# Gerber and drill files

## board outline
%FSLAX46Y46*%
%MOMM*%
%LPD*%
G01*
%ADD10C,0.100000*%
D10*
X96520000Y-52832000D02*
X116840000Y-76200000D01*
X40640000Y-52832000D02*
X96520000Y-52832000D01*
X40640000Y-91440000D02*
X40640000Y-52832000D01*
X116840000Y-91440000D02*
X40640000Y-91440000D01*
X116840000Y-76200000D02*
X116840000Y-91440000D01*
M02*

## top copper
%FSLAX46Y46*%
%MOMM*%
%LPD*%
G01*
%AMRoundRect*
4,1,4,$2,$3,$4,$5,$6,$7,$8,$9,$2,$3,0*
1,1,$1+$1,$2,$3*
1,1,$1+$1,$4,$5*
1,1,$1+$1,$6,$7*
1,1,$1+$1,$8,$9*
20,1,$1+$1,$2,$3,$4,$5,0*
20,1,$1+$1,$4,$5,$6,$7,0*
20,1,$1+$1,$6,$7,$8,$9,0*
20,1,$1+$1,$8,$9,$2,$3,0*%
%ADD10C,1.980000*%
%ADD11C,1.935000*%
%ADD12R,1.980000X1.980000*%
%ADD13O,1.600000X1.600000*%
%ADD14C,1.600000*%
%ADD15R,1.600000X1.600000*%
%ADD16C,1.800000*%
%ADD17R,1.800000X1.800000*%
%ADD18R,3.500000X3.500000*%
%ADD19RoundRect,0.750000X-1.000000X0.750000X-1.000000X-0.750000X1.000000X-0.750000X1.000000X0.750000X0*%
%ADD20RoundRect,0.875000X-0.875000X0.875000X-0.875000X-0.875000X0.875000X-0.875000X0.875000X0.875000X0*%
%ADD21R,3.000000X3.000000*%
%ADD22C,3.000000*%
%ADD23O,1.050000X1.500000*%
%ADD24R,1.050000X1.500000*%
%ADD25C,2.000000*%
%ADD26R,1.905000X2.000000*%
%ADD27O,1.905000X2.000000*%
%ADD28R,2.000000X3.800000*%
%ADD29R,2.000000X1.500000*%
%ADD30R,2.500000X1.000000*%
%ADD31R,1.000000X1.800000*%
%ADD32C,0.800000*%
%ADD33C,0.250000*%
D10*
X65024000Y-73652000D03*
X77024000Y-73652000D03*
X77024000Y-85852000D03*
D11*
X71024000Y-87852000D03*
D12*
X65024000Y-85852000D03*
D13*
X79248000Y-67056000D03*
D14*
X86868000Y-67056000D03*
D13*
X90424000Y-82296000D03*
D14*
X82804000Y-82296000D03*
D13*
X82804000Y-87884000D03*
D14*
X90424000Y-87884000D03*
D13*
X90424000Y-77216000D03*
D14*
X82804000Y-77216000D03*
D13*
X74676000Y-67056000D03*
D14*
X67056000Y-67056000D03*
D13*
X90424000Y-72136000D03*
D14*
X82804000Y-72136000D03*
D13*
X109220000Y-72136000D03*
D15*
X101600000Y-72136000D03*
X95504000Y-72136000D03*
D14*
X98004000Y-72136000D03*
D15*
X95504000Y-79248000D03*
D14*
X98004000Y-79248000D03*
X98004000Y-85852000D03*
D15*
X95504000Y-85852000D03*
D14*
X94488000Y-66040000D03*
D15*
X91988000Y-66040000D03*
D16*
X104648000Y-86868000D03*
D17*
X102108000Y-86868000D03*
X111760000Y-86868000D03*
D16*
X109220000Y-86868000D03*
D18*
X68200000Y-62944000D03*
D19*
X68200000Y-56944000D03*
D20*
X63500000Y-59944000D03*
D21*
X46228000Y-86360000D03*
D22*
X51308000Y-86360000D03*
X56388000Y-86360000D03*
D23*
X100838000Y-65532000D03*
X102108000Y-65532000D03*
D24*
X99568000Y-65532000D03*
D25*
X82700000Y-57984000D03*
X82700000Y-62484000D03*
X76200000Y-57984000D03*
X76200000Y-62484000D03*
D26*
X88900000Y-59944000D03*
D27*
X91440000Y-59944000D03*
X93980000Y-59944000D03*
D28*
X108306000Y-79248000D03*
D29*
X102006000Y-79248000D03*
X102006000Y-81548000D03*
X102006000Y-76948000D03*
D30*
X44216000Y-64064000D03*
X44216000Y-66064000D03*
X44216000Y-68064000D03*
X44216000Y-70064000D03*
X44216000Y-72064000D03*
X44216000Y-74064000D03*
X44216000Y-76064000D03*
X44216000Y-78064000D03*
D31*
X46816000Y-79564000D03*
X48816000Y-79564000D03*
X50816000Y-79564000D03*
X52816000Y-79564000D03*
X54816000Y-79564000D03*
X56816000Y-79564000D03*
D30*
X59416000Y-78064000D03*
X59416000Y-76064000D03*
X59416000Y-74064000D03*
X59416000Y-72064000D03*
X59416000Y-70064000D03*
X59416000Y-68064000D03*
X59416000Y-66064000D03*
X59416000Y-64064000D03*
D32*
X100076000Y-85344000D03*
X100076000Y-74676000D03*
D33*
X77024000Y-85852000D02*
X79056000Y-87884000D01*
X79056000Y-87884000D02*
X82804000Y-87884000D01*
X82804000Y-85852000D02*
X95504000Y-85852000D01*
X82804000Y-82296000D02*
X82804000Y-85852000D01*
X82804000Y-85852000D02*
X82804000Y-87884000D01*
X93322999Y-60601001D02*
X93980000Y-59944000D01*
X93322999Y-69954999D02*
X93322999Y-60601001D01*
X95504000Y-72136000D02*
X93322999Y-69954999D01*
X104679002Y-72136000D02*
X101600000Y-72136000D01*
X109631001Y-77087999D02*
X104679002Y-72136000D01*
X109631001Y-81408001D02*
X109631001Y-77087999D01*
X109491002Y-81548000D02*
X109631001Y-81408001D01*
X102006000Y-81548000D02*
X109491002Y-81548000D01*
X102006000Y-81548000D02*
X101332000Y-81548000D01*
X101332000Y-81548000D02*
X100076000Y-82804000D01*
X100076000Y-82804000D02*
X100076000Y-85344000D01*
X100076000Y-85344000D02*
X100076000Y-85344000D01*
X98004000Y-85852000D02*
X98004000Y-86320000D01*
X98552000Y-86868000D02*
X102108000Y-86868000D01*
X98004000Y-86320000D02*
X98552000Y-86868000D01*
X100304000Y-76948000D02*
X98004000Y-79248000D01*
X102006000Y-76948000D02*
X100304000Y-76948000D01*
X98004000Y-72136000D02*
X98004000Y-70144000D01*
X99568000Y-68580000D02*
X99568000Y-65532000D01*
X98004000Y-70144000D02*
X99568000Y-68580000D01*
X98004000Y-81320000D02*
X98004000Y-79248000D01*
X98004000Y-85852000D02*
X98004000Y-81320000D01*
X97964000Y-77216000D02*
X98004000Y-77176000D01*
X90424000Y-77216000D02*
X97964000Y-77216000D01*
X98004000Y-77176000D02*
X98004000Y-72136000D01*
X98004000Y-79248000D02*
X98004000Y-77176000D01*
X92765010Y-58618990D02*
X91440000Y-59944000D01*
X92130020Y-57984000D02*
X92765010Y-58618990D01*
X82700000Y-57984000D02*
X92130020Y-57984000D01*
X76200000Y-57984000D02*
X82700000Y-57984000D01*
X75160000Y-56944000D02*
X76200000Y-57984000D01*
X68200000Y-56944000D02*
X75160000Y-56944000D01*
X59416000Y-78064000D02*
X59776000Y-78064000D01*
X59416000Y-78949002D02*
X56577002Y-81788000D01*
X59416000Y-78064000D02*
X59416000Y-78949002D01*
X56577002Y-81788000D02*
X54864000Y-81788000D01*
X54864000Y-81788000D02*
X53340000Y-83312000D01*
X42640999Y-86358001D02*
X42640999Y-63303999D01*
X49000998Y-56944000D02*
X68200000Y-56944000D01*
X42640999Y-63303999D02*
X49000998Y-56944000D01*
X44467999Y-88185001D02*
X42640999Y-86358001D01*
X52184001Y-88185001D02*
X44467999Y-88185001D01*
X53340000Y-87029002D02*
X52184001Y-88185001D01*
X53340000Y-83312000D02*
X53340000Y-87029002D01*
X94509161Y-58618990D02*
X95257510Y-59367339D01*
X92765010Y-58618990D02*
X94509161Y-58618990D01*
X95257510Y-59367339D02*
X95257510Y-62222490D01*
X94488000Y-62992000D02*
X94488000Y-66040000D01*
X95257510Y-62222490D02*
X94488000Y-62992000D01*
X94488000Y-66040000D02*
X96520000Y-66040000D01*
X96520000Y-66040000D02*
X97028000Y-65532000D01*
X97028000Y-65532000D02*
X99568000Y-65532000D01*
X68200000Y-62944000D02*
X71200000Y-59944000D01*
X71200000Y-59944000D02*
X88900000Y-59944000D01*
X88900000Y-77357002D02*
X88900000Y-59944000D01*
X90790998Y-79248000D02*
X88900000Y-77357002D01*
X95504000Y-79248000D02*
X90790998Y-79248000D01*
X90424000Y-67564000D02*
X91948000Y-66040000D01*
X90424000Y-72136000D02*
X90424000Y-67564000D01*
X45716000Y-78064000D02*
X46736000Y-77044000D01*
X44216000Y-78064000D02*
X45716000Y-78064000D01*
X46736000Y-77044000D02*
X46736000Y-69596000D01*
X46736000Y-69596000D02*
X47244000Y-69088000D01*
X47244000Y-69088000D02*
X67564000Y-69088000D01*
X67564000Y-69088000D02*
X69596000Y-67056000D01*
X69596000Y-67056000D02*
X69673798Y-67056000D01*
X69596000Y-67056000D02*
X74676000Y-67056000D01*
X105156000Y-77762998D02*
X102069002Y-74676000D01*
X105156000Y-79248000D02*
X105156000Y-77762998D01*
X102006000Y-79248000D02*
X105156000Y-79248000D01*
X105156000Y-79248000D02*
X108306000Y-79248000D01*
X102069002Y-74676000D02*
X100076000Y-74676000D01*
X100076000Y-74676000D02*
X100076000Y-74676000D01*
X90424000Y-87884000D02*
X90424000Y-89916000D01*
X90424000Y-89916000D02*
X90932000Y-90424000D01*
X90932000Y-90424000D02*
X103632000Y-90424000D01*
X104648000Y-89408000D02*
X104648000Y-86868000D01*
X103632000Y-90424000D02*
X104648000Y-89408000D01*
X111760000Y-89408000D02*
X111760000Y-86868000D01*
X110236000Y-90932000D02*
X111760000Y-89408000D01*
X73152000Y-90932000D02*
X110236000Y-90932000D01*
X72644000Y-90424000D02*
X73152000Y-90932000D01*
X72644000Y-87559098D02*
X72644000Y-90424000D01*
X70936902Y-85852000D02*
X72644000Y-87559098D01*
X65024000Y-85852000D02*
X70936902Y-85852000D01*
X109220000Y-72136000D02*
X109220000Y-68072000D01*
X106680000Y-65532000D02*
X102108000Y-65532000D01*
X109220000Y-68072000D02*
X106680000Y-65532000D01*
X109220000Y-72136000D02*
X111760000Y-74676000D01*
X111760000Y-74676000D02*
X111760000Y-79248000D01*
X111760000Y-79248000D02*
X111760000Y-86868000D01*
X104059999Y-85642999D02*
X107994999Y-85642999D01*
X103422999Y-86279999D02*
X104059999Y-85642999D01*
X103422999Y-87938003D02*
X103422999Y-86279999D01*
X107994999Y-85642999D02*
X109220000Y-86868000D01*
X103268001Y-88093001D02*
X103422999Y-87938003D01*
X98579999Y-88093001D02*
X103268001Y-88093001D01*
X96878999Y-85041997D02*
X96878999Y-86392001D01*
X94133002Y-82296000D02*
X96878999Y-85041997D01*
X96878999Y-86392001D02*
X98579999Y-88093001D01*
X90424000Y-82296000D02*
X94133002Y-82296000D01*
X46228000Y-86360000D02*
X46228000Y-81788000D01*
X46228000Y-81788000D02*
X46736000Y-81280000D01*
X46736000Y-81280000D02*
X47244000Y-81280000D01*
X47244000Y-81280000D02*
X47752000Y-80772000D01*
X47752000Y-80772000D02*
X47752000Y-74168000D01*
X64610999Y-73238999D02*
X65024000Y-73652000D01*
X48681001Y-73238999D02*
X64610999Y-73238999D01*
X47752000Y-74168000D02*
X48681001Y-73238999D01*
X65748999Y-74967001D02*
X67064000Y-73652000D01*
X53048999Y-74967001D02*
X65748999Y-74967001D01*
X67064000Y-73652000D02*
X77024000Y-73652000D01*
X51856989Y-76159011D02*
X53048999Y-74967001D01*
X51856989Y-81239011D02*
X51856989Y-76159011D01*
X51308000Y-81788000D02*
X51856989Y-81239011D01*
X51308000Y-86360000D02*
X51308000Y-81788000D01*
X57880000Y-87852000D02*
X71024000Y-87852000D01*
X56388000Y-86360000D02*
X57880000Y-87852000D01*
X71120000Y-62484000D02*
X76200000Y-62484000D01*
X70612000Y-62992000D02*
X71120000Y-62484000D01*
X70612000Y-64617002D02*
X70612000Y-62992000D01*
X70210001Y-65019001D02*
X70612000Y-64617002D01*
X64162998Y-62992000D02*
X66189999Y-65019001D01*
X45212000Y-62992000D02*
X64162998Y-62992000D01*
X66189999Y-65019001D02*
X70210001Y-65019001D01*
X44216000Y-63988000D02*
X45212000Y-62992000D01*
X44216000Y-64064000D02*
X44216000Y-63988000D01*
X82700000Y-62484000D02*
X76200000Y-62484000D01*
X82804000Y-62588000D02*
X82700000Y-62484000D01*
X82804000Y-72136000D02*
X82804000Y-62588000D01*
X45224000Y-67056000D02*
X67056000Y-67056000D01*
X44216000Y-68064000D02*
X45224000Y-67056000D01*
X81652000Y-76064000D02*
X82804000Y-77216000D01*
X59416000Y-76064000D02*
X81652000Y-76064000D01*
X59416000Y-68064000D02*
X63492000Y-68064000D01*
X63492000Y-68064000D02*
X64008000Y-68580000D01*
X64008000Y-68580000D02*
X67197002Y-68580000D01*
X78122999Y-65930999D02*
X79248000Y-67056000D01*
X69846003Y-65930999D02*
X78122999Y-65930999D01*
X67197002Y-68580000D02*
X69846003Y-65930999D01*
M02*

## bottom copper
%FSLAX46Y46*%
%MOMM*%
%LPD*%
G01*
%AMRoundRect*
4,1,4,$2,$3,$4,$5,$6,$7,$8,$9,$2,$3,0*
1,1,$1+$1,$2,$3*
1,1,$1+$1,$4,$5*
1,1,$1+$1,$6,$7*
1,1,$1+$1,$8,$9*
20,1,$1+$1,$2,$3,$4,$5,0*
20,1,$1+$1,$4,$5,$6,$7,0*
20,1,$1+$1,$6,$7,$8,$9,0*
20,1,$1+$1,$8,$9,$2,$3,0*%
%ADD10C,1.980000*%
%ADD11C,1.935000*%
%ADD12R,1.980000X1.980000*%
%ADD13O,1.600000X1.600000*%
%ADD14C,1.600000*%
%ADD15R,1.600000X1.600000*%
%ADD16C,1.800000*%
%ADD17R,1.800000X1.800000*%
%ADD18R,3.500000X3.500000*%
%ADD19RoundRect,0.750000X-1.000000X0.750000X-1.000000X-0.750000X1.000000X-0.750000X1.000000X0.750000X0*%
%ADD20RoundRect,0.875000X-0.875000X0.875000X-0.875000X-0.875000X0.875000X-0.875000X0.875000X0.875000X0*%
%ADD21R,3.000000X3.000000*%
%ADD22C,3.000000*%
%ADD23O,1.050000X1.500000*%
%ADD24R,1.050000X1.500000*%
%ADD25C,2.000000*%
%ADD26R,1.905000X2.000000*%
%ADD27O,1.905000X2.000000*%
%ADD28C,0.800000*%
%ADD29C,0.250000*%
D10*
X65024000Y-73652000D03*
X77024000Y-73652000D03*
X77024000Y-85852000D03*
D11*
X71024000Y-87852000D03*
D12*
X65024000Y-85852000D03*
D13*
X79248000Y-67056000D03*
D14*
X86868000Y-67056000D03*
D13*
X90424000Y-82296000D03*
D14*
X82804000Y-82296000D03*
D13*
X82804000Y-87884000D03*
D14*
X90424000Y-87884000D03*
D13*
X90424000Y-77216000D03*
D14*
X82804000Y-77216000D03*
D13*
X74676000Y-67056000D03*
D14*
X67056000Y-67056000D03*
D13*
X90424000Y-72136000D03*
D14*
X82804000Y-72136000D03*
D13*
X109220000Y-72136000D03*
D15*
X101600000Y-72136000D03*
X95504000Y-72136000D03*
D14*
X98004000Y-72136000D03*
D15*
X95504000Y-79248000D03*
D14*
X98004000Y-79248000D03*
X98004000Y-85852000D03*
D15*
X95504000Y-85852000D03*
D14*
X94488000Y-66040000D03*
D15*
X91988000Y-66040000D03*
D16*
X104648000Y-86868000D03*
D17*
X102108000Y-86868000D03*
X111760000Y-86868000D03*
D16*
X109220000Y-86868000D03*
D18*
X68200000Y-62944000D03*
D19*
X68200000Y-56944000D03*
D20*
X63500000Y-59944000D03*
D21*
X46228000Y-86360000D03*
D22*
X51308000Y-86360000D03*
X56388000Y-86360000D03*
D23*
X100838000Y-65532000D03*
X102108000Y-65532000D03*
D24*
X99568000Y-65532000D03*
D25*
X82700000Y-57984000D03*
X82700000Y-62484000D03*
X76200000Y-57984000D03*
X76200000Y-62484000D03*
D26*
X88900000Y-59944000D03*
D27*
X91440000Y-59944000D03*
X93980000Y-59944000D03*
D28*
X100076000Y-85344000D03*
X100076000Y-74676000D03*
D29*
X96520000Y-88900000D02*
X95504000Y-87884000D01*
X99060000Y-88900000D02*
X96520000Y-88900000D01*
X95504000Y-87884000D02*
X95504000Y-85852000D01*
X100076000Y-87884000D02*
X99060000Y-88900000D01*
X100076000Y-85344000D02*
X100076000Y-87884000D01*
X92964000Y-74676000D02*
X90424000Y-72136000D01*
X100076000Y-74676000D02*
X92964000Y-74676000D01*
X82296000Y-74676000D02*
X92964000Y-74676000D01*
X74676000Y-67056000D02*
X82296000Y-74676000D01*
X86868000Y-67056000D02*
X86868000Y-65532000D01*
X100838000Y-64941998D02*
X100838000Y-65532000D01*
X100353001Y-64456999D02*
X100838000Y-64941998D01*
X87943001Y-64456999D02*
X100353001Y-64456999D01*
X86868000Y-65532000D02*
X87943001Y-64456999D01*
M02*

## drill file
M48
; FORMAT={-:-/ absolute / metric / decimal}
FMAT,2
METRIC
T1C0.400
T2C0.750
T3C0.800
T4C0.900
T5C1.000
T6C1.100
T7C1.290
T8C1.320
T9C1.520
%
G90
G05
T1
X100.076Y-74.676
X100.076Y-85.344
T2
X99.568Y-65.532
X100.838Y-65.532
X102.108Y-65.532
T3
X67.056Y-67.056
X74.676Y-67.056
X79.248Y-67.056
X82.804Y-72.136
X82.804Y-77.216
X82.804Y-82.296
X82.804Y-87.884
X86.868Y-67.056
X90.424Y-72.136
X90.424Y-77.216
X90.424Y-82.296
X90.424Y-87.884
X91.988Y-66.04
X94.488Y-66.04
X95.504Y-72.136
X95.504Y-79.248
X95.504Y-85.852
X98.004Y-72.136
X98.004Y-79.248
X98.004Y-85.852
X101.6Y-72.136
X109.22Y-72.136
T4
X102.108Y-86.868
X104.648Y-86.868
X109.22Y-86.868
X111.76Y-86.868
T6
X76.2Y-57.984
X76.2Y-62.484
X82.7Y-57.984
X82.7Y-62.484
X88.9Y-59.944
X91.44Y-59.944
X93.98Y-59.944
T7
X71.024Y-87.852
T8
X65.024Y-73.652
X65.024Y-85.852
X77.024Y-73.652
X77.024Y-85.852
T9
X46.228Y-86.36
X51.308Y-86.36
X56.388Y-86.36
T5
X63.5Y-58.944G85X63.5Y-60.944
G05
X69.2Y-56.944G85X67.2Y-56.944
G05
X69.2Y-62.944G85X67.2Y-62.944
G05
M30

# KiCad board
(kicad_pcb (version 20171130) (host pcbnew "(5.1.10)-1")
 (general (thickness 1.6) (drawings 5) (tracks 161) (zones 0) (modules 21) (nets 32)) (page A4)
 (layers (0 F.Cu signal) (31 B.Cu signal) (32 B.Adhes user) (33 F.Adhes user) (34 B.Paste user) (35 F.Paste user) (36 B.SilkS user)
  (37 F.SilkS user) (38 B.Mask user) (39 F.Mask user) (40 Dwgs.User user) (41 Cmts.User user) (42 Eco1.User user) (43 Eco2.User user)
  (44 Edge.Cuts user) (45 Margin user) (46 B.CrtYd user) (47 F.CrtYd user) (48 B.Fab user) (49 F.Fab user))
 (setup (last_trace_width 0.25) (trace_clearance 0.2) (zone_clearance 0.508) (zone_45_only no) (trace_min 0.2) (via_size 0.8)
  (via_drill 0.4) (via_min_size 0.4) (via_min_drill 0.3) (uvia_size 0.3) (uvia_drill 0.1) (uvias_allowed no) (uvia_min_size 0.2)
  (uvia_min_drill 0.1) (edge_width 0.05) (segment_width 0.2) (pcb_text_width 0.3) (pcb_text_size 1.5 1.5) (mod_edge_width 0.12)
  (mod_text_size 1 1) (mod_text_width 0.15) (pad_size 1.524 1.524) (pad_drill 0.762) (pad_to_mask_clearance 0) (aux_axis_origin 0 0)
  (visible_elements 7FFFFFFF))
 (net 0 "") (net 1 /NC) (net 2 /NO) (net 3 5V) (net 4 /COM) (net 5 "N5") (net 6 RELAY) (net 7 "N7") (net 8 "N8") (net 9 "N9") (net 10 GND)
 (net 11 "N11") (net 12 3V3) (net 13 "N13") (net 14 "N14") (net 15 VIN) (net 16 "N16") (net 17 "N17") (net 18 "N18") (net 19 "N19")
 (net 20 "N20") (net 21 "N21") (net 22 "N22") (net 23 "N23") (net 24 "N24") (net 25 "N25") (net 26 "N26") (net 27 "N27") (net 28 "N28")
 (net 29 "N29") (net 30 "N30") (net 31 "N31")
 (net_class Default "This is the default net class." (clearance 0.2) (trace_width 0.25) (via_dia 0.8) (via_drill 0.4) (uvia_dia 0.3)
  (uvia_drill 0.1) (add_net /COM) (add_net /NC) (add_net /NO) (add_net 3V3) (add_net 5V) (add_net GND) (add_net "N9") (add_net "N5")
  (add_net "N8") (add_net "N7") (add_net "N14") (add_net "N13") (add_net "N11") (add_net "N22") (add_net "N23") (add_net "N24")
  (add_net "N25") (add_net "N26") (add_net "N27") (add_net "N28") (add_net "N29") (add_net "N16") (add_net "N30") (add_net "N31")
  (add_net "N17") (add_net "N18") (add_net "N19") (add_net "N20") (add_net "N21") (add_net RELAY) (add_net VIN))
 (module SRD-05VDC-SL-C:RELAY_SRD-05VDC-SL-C (layer F.Cu) (at 71.024 79.752 90)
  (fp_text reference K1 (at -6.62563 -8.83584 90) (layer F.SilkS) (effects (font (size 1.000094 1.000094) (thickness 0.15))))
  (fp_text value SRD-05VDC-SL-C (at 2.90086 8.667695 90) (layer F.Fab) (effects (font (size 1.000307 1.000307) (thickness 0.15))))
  (pad NC thru_hole circle (at 6.1 -6 90) (size 1.98 1.98) (drill 1.32) (layers *.Cu *.Mask) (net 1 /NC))
  (pad NO thru_hole circle (at 6.1 6 90) (size 1.98 1.98) (drill 1.32) (layers *.Cu *.Mask) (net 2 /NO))
  (pad A2 thru_hole circle (at -6.1 6 90) (size 1.98 1.98) (drill 1.32) (layers *.Cu *.Mask) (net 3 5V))
  (pad COM thru_hole circle (at -8.1 0 90) (size 1.935 1.935) (drill 1.29) (layers *.Cu *.Mask) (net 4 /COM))
  (pad A1 thru_hole rect (at -6.1 -6 90) (size 1.98 1.98) (drill 1.32) (layers *.Cu *.Mask) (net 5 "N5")))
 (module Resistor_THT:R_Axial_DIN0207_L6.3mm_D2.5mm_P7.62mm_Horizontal (layer F.Cu) (at 86.868 67.056 180)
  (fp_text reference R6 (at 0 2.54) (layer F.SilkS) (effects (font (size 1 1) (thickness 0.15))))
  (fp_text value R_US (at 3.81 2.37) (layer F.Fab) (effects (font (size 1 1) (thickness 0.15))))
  (pad 2 thru_hole oval (at 7.62 0 180) (size 1.6 1.6) (drill 0.8) (layers *.Cu *.Mask) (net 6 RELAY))
  (pad 1 thru_hole circle (at 0 0 180) (size 1.6 1.6) (drill 0.8) (layers *.Cu *.Mask) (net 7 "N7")))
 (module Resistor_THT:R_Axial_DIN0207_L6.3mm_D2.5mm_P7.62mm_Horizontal (layer F.Cu) (at 82.804 82.296)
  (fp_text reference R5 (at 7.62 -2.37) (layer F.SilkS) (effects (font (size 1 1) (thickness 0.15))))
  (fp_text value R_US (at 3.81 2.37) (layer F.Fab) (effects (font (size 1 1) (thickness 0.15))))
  (pad 2 thru_hole oval (at 7.62 0) (size 1.6 1.6) (drill 0.8) (layers *.Cu *.Mask) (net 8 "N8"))
  (pad 1 thru_hole circle (at 0 0) (size 1.6 1.6) (drill 0.8) (layers *.Cu *.Mask) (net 3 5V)))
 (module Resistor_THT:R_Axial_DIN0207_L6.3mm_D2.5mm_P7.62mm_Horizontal (layer F.Cu) (at 90.424 87.884 180)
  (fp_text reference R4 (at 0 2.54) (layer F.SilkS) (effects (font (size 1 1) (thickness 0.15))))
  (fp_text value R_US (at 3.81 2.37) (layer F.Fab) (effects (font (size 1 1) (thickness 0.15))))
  (pad 2 thru_hole oval (at 7.62 0 180) (size 1.6 1.6) (drill 0.8) (layers *.Cu *.Mask) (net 3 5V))
  (pad 1 thru_hole circle (at 0 0 180) (size 1.6 1.6) (drill 0.8) (layers *.Cu *.Mask) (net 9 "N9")))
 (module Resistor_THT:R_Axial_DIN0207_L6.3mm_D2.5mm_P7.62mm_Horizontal (layer F.Cu) (at 82.804 77.216)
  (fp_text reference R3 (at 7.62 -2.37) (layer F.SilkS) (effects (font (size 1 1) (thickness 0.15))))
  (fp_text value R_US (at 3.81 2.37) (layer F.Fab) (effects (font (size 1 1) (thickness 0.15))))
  (pad 2 thru_hole oval (at 7.62 0) (size 1.6 1.6) (drill 0.8) (layers *.Cu *.Mask) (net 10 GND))
  (pad 1 thru_hole circle (at 0 0) (size 1.6 1.6) (drill 0.8) (layers *.Cu *.Mask) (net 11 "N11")))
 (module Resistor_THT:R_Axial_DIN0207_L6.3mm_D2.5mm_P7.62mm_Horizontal (layer F.Cu) (at 67.056 67.056)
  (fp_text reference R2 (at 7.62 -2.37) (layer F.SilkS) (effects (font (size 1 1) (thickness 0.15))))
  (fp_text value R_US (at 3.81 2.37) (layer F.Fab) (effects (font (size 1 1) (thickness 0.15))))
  (pad 2 thru_hole oval (at 7.62 0) (size 1.6 1.6) (drill 0.8) (layers *.Cu *.Mask) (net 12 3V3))
  (pad 1 thru_hole circle (at 0 0) (size 1.6 1.6) (drill 0.8) (layers *.Cu *.Mask) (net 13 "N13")))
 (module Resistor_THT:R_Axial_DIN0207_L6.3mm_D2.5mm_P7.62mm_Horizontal (layer F.Cu) (at 82.804 72.136)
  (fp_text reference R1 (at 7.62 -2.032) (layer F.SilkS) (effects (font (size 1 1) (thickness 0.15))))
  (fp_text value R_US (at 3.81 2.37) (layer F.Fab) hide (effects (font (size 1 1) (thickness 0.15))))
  (pad 2 thru_hole oval (at 7.62 0) (size 1.6 1.6) (drill 0.8) (layers *.Cu *.Mask) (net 12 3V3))
  (pad 1 thru_hole circle (at 0 0) (size 1.6 1.6) (drill 0.8) (layers *.Cu *.Mask) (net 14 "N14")))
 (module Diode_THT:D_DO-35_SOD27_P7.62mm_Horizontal (layer F.Cu) (at 101.6 72.136)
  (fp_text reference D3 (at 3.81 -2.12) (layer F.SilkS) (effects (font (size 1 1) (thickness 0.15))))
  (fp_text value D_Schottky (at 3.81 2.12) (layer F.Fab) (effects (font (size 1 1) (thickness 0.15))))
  (pad 2 thru_hole oval (at 7.62 0) (size 1.6 1.6) (drill 0.8) (layers *.Cu *.Mask) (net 5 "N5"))
  (pad 1 thru_hole rect (at 0 0) (size 1.6 1.6) (drill 0.8) (layers *.Cu *.Mask) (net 3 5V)))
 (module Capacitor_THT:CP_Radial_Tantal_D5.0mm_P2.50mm (layer F.Cu) (at 95.504 72.136)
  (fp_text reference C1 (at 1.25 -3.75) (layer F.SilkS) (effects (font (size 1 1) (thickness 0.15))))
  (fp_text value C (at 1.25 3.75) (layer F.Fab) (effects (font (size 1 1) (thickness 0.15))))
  (pad 1 thru_hole rect (at 0 0) (size 1.6 1.6) (drill 0.8) (layers *.Cu *.Mask) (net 3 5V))
  (pad 2 thru_hole circle (at 2.5 0) (size 1.6 1.6) (drill 0.8) (layers *.Cu *.Mask) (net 10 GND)))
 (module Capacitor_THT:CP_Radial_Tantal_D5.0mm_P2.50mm (layer F.Cu) (at 95.504 79.248)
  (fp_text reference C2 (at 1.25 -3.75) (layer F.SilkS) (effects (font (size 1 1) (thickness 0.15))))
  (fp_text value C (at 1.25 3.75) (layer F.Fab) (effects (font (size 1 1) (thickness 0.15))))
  (pad 1 thru_hole rect (at 0 0) (size 1.6 1.6) (drill 0.8) (layers *.Cu *.Mask) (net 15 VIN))
  (pad 2 thru_hole circle (at 2.5 0) (size 1.6 1.6) (drill 0.8) (layers *.Cu *.Mask) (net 10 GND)))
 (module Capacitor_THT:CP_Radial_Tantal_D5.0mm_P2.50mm (layer F.Cu) (at 95.504 85.852)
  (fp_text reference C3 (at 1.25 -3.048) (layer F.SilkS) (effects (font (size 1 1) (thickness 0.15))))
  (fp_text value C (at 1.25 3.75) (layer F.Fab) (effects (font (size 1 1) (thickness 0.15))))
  (pad 2 thru_hole circle (at 2.5 0) (size 1.6 1.6) (drill 0.8) (layers *.Cu *.Mask) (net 10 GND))
  (pad 1 thru_hole rect (at 0 0) (size 1.6 1.6) (drill 0.8) (layers *.Cu *.Mask) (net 3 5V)))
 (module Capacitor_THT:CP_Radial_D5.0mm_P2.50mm (layer F.Cu) (at 91.988 66.04)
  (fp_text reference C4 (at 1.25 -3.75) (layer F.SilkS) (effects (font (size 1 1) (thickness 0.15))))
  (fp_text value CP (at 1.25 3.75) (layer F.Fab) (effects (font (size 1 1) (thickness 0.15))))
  (pad 2 thru_hole circle (at 2.5 0) (size 1.6 1.6) (drill 0.8) (layers *.Cu *.Mask) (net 10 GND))
  (pad 1 thru_hole rect (at 0 0) (size 1.6 1.6) (drill 0.8) (layers *.Cu *.Mask) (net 12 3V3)))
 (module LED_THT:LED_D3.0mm (layer F.Cu) (at 102.108 86.868)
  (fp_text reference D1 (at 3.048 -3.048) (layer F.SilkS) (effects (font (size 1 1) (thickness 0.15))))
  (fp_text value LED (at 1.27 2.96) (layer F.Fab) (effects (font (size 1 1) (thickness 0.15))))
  (pad 2 thru_hole circle (at 2.54 0) (size 1.8 1.8) (drill 0.9) (layers *.Cu *.Mask) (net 9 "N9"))
  (pad 1 thru_hole rect (at 0 0) (size 1.8 1.8) (drill 0.9) (layers *.Cu *.Mask) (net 10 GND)))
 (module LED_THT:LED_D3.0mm (layer F.Cu) (at 111.76 86.868 180)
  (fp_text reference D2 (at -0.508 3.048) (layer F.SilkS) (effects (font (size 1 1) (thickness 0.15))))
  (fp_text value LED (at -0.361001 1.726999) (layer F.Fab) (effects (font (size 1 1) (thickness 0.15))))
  (pad 1 thru_hole rect (at 0 0 180) (size 1.8 1.8) (drill 0.9) (layers *.Cu *.Mask) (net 5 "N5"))
  (pad 2 thru_hole circle (at 2.54 0 180) (size 1.8 1.8) (drill 0.9) (layers *.Cu *.Mask) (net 8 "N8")))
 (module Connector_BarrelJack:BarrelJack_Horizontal (layer F.Cu) (at 68.2 62.944 270)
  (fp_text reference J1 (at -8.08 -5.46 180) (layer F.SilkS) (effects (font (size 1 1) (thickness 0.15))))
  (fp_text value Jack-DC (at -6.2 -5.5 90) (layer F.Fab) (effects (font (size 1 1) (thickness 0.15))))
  (pad 1 thru_hole rect (at 0 0 270) (size 3.5 3.5) (drill oval 1 3) (layers *.Cu *.Mask) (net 15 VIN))
  (pad 2 thru_hole roundrect (at -6 0 270) (size 3 3.5) (drill oval 1 3) (layers *.Cu *.Mask) (roundrect_rratio 0.25) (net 10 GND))
  (pad 3 thru_hole roundrect (at -3 4.7 270) (size 3.5 3.5) (drill oval 3 1) (layers *.Cu *.Mask) (roundrect_rratio 0.25)))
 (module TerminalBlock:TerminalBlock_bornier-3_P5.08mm (layer F.Cu) (at 46.228 86.36)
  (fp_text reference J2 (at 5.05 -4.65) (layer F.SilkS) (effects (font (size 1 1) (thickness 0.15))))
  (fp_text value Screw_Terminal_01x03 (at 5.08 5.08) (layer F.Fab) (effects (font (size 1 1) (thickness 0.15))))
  (pad 1 thru_hole rect (at 0 0) (size 3 3) (drill 1.52) (layers *.Cu *.Mask) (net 1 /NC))
  (pad 2 thru_hole circle (at 5.08 0) (size 3 3) (drill 1.52) (layers *.Cu *.Mask) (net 2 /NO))
  (pad 3 thru_hole circle (at 10.16 0) (size 3 3) (drill 1.52) (layers *.Cu *.Mask) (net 4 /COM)))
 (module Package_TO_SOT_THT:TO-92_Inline (layer F.Cu) (at 99.568 65.532)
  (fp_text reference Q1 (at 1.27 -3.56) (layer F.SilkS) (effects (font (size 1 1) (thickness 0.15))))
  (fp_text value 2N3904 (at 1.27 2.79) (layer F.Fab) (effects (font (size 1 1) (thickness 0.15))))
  (pad 2 thru_hole oval (at 1.27 0) (size 1.05 1.5) (drill 0.75) (layers *.Cu *.Mask) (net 7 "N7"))
  (pad 3 thru_hole oval (at 2.54 0) (size 1.05 1.5) (drill 0.75) (layers *.Cu *.Mask) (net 5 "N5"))
  (pad 1 thru_hole rect (at 0 0) (size 1.05 1.5) (drill 0.75) (layers *.Cu *.Mask) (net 10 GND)))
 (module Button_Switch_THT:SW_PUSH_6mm (layer F.Cu) (at 82.7 62.484 180)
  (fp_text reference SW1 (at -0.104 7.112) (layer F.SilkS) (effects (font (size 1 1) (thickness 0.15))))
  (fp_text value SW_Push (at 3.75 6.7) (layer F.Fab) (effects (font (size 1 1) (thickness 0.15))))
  (pad 2 thru_hole circle (at 0 4.5 270) (size 2 2) (drill 1.1) (layers *.Cu *.Mask) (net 10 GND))
  (pad 1 thru_hole circle (at 0 0 270) (size 2 2) (drill 1.1) (layers *.Cu *.Mask) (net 14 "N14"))
  (pad 2 thru_hole circle (at 6.5 4.5 270) (size 2 2) (drill 1.1) (layers *.Cu *.Mask) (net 10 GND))
  (pad 1 thru_hole circle (at 6.5 0 270) (size 2 2) (drill 1.1) (layers *.Cu *.Mask) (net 14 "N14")))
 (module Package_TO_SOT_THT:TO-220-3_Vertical (layer F.Cu) (at 88.9 59.944)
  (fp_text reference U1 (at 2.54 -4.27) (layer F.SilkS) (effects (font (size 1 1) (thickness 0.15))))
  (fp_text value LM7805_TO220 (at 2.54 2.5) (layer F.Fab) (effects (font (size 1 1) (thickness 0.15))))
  (pad 1 thru_hole rect (at 0 0) (size 1.905 2) (drill 1.1) (layers *.Cu *.Mask) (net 15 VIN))
  (pad 2 thru_hole oval (at 2.54 0) (size 1.905 2) (drill 1.1) (layers *.Cu *.Mask) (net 10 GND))
  (pad 3 thru_hole oval (at 5.08 0) (size 1.905 2) (drill 1.1) (layers *.Cu *.Mask) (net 3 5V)))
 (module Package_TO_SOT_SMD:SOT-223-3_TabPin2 (layer F.Cu) (at 105.156 79.248)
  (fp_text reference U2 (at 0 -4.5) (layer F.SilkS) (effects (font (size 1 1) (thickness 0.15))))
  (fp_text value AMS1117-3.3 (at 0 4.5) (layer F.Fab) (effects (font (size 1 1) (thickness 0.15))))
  (pad 2 smd rect (at 3.15 0) (size 2 3.8) (layers F.Cu F.Paste F.Mask) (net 12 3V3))
  (pad 2 smd rect (at -3.15 0) (size 2 1.5) (layers F.Cu F.Paste F.Mask) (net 12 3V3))
  (pad 3 smd rect (at -3.15 2.3) (size 2 1.5) (layers F.Cu F.Paste F.Mask) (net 3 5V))
  (pad 1 smd rect (at -3.15 -2.3) (size 2 1.5) (layers F.Cu F.Paste F.Mask) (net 10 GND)))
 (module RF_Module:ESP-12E (layer F.Cu) (at 51.816 67.564)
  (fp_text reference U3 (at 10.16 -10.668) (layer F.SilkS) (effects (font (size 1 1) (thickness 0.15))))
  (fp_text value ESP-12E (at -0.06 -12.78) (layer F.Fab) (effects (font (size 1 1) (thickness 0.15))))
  (pad 1 smd rect (at -7.6 -3.5) (size 2.5 1) (layers F.Cu F.Paste F.Mask) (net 14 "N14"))
  (pad 2 smd rect (at -7.6 -1.5) (size 2.5 1) (layers F.Cu F.Paste F.Mask) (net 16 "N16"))
  (pad 3 smd rect (at -7.6 0.5) (size 2.5 1) (layers F.Cu F.Paste F.Mask) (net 13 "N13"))
  (pad 4 smd rect (at -7.6 2.5) (size 2.5 1) (layers F.Cu F.Paste F.Mask) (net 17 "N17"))
  (pad 5 smd rect (at -7.6 4.5) (size 2.5 1) (layers F.Cu F.Paste F.Mask) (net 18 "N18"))
  (pad 6 smd rect (at -7.6 6.5) (size 2.5 1) (layers F.Cu F.Paste F.Mask) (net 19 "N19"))
  (pad 7 smd rect (at -7.6 8.5) (size 2.5 1) (layers F.Cu F.Paste F.Mask) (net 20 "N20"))
  (pad 8 smd rect (at -7.6 10.5) (size 2.5 1) (layers F.Cu F.Paste F.Mask) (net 12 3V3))
  (pad 9 smd rect (at -5 12) (size 1 1.8) (layers F.Cu F.Paste F.Mask) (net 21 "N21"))
  (pad 10 smd rect (at -3 12) (size 1 1.8) (layers F.Cu F.Paste F.Mask) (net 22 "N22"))
  (pad 11 smd rect (at -1 12) (size 1 1.8) (layers F.Cu F.Paste F.Mask) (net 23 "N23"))
  (pad 12 smd rect (at 1 12) (size 1 1.8) (layers F.Cu F.Paste F.Mask) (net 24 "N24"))
  (pad 13 smd rect (at 3 12) (size 1 1.8) (layers F.Cu F.Paste F.Mask) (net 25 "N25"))
  (pad 14 smd rect (at 5 12) (size 1 1.8) (layers F.Cu F.Paste F.Mask) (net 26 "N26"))
  (pad 15 smd rect (at 7.6 10.5) (size 2.5 1) (layers F.Cu F.Paste F.Mask) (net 10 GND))
  (pad 16 smd rect (at 7.6 8.5) (size 2.5 1) (layers F.Cu F.Paste F.Mask) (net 11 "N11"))
  (pad 17 smd rect (at 7.6 6.5) (size 2.5 1) (layers F.Cu F.Paste F.Mask) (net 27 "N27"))
  (pad 18 smd rect (at 7.6 4.5) (size 2.5 1) (layers F.Cu F.Paste F.Mask) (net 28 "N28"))
  (pad 19 smd rect (at 7.6 2.5) (size 2.5 1) (layers F.Cu F.Paste F.Mask) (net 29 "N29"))
  (pad 20 smd rect (at 7.6 0.5) (size 2.5 1) (layers F.Cu F.Paste F.Mask) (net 6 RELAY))
  (pad 21 smd rect (at 7.6 -1.5) (size 2.5 1) (layers F.Cu F.Paste F.Mask) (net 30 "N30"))
  (pad 22 smd rect (at 7.6 -3.5) (size 2.5 1) (layers F.Cu F.Paste F.Mask) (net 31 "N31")))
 (gr_line (start 96.52 52.832) (end 116.84 76.2) (layer Edge.Cuts) (width 0.1))
 (gr_line (start 40.64 52.832) (end 96.52 52.832) (layer Edge.Cuts) (width 0.1))
 (gr_line (start 40.64 91.44) (end 40.64 52.832) (layer Edge.Cuts) (width 0.1))
 (gr_line (start 116.84 91.44) (end 40.64 91.44) (layer Edge.Cuts) (width 0.1))
 (gr_line (start 116.84 76.2) (end 116.84 91.44) (layer Edge.Cuts) (width 0.1))
 (segment (start 77.024 85.852) (end 79.056 87.884) (width 0.25) (layer F.Cu) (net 3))
 (segment (start 79.056 87.884) (end 82.804 87.884) (width 0.25) (layer F.Cu) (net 3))
 (segment (start 82.804 85.852) (end 95.504 85.852) (width 0.25) (layer F.Cu) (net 3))
 (segment (start 82.804 82.296) (end 82.804 85.852) (width 0.25) (layer F.Cu) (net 3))
 (segment (start 82.804 85.852) (end 82.804 87.884) (width 0.25) (layer F.Cu) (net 3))
 (segment (start 93.322999 60.601001) (end 93.98 59.944) (width 0.25) (layer F.Cu) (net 3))
 (segment (start 93.322999 69.954999) (end 93.322999 60.601001) (width 0.25) (layer F.Cu) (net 3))
 (segment (start 95.504 72.136) (end 93.322999 69.954999) (width 0.25) (layer F.Cu) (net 3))
 (segment (start 104.679002 72.136) (end 101.6 72.136) (width 0.25) (layer F.Cu) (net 3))
 (segment (start 109.631001 77.087999) (end 104.679002 72.136) (width 0.25) (layer F.Cu) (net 3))
 (segment (start 109.631001 81.408001) (end 109.631001 77.087999) (width 0.25) (layer F.Cu) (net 3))
 (segment (start 109.491002 81.548) (end 109.631001 81.408001) (width 0.25) (layer F.Cu) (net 3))
 (segment (start 102.006 81.548) (end 109.491002 81.548) (width 0.25) (layer F.Cu) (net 3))
 (segment (start 102.006 81.548) (end 101.332 81.548) (width 0.25) (layer F.Cu) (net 3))
 (segment (start 101.332 81.548) (end 100.076 82.804) (width 0.25) (layer F.Cu) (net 3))
 (segment (start 100.076 82.804) (end 100.076 85.344) (width 0.25) (layer F.Cu) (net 3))
 (segment (start 100.076 85.344) (end 100.076 85.344) (width 0.25) (layer F.Cu) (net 3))
 (via (at 100.076 85.344) (size 0.8) (drill 0.4) (layers F.Cu B.Cu) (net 3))
 (segment (start 96.52 88.9) (end 95.504 87.884) (width 0.25) (layer B.Cu) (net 3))
 (segment (start 99.06 88.9) (end 96.52 88.9) (width 0.25) (layer B.Cu) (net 3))
 (segment (start 95.504 87.884) (end 95.504 85.852) (width 0.25) (layer B.Cu) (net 3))
 (segment (start 100.076 87.884) (end 99.06 88.9) (width 0.25) (layer B.Cu) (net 3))
 (segment (start 100.076 85.344) (end 100.076 87.884) (width 0.25) (layer B.Cu) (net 3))
 (segment (start 98.004 85.852) (end 98.004 86.32) (width 0.25) (layer F.Cu) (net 10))
 (segment (start 98.552 86.868) (end 102.108 86.868) (width 0.25) (layer F.Cu) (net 10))
 (segment (start 98.004 86.32) (end 98.552 86.868) (width 0.25) (layer F.Cu) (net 10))
 (segment (start 100.304 76.948) (end 98.004 79.248) (width 0.25) (layer F.Cu) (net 10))
 (segment (start 102.006 76.948) (end 100.304 76.948) (width 0.25) (layer F.Cu) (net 10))
 (segment (start 98.004 72.136) (end 98.004 70.144) (width 0.25) (layer F.Cu) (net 10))
 (segment (start 99.568 68.58) (end 99.568 65.532) (width 0.25) (layer F.Cu) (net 10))
 (segment (start 98.004 70.144) (end 99.568 68.58) (width 0.25) (layer F.Cu) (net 10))
 (segment (start 98.004 81.32) (end 98.004 79.248) (width 0.25) (layer F.Cu) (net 10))
 (segment (start 98.004 85.852) (end 98.004 81.32) (width 0.25) (layer F.Cu) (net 10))
 (segment (start 97.964 77.216) (end 98.004 77.176) (width 0.25) (layer F.Cu) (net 10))
 (segment (start 90.424 77.216) (end 97.964 77.216) (width 0.25) (layer F.Cu) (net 10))
 (segment (start 98.004 77.176) (end 98.004 72.136) (width 0.25) (layer F.Cu) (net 10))
 (segment (start 98.004 79.248) (end 98.004 77.176) (width 0.25) (layer F.Cu) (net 10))
 (segment (start 92.76501 58.61899) (end 91.44 59.944) (width 0.25) (layer F.Cu) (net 10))
 (segment (start 92.13002 57.984) (end 92.76501 58.61899) (width 0.25) (layer F.Cu) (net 10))
 (segment (start 82.7 57.984) (end 92.13002 57.984) (width 0.25) (layer F.Cu) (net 10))
 (segment (start 76.2 57.984) (end 82.7 57.984) (width 0.25) (layer F.Cu) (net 10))
 (segment (start 75.16 56.944) (end 76.2 57.984) (width 0.25) (layer F.Cu) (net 10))
 (segment (start 68.2 56.944) (end 75.16 56.944) (width 0.25) (layer F.Cu) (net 10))
 (segment (start 59.416 78.064) (end 59.776 78.064) (width 0.25) (layer F.Cu) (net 10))
 (segment (start 59.416 78.949002) (end 56.577002 81.788) (width 0.25) (layer F.Cu) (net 10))
 (segment (start 59.416 78.064) (end 59.416 78.949002) (width 0.25) (layer F.Cu) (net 10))
 (segment (start 56.577002 81.788) (end 54.864 81.788) (width 0.25) (layer F.Cu) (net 10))
 (segment (start 54.864 81.788) (end 53.34 83.312) (width 0.25) (layer F.Cu) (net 10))
 (segment (start 42.640999 86.358001) (end 42.640999 63.303999) (width 0.25) (layer F.Cu) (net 10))
 (segment (start 49.000998 56.944) (end 68.2 56.944) (width 0.25) (layer F.Cu) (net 10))
 (segment (start 42.640999 63.303999) (end 49.000998 56.944) (width 0.25) (layer F.Cu) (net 10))
 (segment (start 44.467999 88.185001) (end 42.640999 86.358001) (width 0.25) (layer F.Cu) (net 10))
 (segment (start 52.184001 88.185001) (end 44.467999 88.185001) (width 0.25) (layer F.Cu) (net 10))
 (segment (start 53.34 87.029002) (end 52.184001 88.185001) (width 0.25) (layer F.Cu) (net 10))
 (segment (start 53.34 83.312) (end 53.34 87.029002) (width 0.25) (layer F.Cu) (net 10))
 (segment (start 94.509161 58.61899) (end 95.25751 59.367339) (width 0.25) (layer F.Cu) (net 10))
 (segment (start 92.76501 58.61899) (end 94.509161 58.61899) (width 0.25) (layer F.Cu) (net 10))
 (segment (start 95.25751 59.367339) (end 95.25751 62.22249) (width 0.25) (layer F.Cu) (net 10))
 (segment (start 94.488 62.992) (end 94.488 66.04) (width 0.25) (layer F.Cu) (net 10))
 (segment (start 95.25751 62.22249) (end 94.488 62.992) (width 0.25) (layer F.Cu) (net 10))
 (segment (start 94.488 66.04) (end 96.52 66.04) (width 0.25) (layer F.Cu) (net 10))
 (segment (start 96.52 66.04) (end 97.028 65.532) (width 0.25) (layer F.Cu) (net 10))
 (segment (start 97.028 65.532) (end 99.568 65.532) (width 0.25) (layer F.Cu) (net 10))
 (segment (start 68.2 62.944) (end 71.2 59.944) (width 0.25) (layer F.Cu) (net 15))
 (segment (start 71.2 59.944) (end 88.9 59.944) (width 0.25) (layer F.Cu) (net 15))
 (segment (start 88.9 77.357002) (end 88.9 59.944) (width 0.25) (layer F.Cu) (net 15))
 (segment (start 90.790998 79.248) (end 88.9 77.357002) (width 0.25) (layer F.Cu) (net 15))
 (segment (start 95.504 79.248) (end 90.790998 79.248) (width 0.25) (layer F.Cu) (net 15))
 (segment (start 90.424 67.564) (end 91.948 66.04) (width 0.25) (layer F.Cu) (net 12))
 (segment (start 90.424 72.136) (end 90.424 67.564) (width 0.25) (layer F.Cu) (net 12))
 (segment (start 45.716 78.064) (end 46.736 77.044) (width 0.25) (layer F.Cu) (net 12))
 (segment (start 44.216 78.064) (end 45.716 78.064) (width 0.25) (layer F.Cu) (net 12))
 (segment (start 46.736 77.044) (end 46.736 69.596) (width 0.25) (layer F.Cu) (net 12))
 (segment (start 46.736 69.596) (end 47.244 69.088) (width 0.25) (layer F.Cu) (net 12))
 (segment (start 47.244 69.088) (end 67.564 69.088) (width 0.25) (layer F.Cu) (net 12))
 (segment (start 67.564 69.088) (end 69.596 67.056) (width 0.25) (layer F.Cu) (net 12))
 (segment (start 69.596 67.056) (end 69.673798 67.056) (width 0.25) (layer F.Cu) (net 12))
 (segment (start 69.596 67.056) (end 74.676 67.056) (width 0.25) (layer F.Cu) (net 12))
 (segment (start 105.156 77.762998) (end 102.069002 74.676) (width 0.25) (layer F.Cu) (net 12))
 (segment (start 105.156 79.248) (end 105.156 77.762998) (width 0.25) (layer F.Cu) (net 12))
 (segment (start 102.006 79.248) (end 105.156 79.248) (width 0.25) (layer F.Cu) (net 12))
 (segment (start 105.156 79.248) (end 108.306 79.248) (width 0.25) (layer F.Cu) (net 12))
 (segment (start 102.069002 74.676) (end 100.076 74.676) (width 0.25) (layer F.Cu) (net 12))
 (segment (start 100.076 74.676) (end 100.076 74.676) (width 0.25) (layer F.Cu) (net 12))
 (via (at 100.076 74.676) (size 0.8) (drill 0.4) (layers F.Cu B.Cu) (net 12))
 (segment (start 92.964 74.676) (end 90.424 72.136) (width 0.25) (layer B.Cu) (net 12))
 (segment (start 100.076 74.676) (end 92.964 74.676) (width 0.25) (layer B.Cu) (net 12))
 (segment (start 82.296 74.676) (end 92.964 74.676) (width 0.25) (layer B.Cu) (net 12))
 (segment (start 74.676 67.056) (end 82.296 74.676) (width 0.25) (layer B.Cu) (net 12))
 (segment (start 90.424 87.884) (end 90.424 89.916) (width 0.25) (layer F.Cu) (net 9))
 (segment (start 90.424 89.916) (end 90.932 90.424) (width 0.25) (layer F.Cu) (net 9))
 (segment (start 90.932 90.424) (end 103.632 90.424) (width 0.25) (layer F.Cu) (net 9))
 (segment (start 104.648 89.408) (end 104.648 86.868) (width 0.25) (layer F.Cu) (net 9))
 (segment (start 103.632 90.424) (end 104.648 89.408) (width 0.25) (layer F.Cu) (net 9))
 (segment (start 111.76 89.408) (end 111.76 86.868) (width 0.25) (layer F.Cu) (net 5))
 (segment (start 110.236 90.932) (end 111.76 89.408) (width 0.25) (layer F.Cu) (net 5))
 (segment (start 73.152 90.932) (end 110.236 90.932) (width 0.25) (layer F.Cu) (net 5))
 (segment (start 72.644 90.424) (end 73.152 90.932) (width 0.25) (layer F.Cu) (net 5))
 (segment (start 72.644 87.559098) (end 72.644 90.424) (width 0.25) (layer F.Cu) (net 5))
 (segment (start 70.936902 85.852) (end 72.644 87.559098) (width 0.25) (layer F.Cu) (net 5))
 (segment (start 65.024 85.852) (end 70.936902 85.852) (width 0.25) (layer F.Cu) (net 5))
 (segment (start 109.22 72.136) (end 109.22 68.072) (width 0.25) (layer F.Cu) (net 5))
 (segment (start 106.68 65.532) (end 102.108 65.532) (width 0.25) (layer F.Cu) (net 5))
 (segment (start 109.22 68.072) (end 106.68 65.532) (width 0.25) (layer F.Cu) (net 5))
 (segment (start 109.22 72.136) (end 111.76 74.676) (width 0.25) (layer F.Cu) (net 5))
 (segment (start 111.76 74.676) (end 111.76 79.248) (width 0.25) (layer F.Cu) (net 5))
 (segment (start 111.76 79.248) (end 111.76 86.868) (width 0.25) (layer F.Cu) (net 5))
 (segment (start 104.059999 85.642999) (end 107.994999 85.642999) (width 0.25) (layer F.Cu) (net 8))
 (segment (start 103.422999 86.279999) (end 104.059999 85.642999) (width 0.25) (layer F.Cu) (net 8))
 (segment (start 103.422999 87.938003) (end 103.422999 86.279999) (width 0.25) (layer F.Cu) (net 8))
 (segment (start 107.994999 85.642999) (end 109.22 86.868) (width 0.25) (layer F.Cu) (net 8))
 (segment (start 103.268001 88.093001) (end 103.422999 87.938003) (width 0.25) (layer F.Cu) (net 8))
 (segment (start 98.579999 88.093001) (end 103.268001 88.093001) (width 0.25) (layer F.Cu) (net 8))
 (segment (start 96.878999 85.041997) (end 96.878999 86.392001) (width 0.25) (layer F.Cu) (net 8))
 (segment (start 94.133002 82.296) (end 96.878999 85.041997) (width 0.25) (layer F.Cu) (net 8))
 (segment (start 96.878999 86.392001) (end 98.579999 88.093001) (width 0.25) (layer F.Cu) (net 8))
 (segment (start 90.424 82.296) (end 94.133002 82.296) (width 0.25) (layer F.Cu) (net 8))
 (segment (start 46.228 86.36) (end 46.228 81.788) (width 0.25) (layer F.Cu) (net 1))
 (segment (start 46.228 81.788) (end 46.736 81.28) (width 0.25) (layer F.Cu) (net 1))
 (segment (start 46.736 81.28) (end 47.244 81.28) (width 0.25) (layer F.Cu) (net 1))
 (segment (start 47.244 81.28) (end 47.752 80.772) (width 0.25) (layer F.Cu) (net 1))
 (segment (start 47.752 80.772) (end 47.752 74.168) (width 0.25) (layer F.Cu) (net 1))
 (segment (start 64.610999 73.238999) (end 65.024 73.652) (width 0.25) (layer F.Cu) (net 1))
 (segment (start 48.681001 73.238999) (end 64.610999 73.238999) (width 0.25) (layer F.Cu) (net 1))
 (segment (start 47.752 74.168) (end 48.681001 73.238999) (width 0.25) (layer F.Cu) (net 1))
 (segment (start 65.748999 74.967001) (end 67.064 73.652) (width 0.25) (layer F.Cu) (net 2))
 (segment (start 53.048999 74.967001) (end 65.748999 74.967001) (width 0.25) (layer F.Cu) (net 2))
 (segment (start 67.064 73.652) (end 77.024 73.652) (width 0.25) (layer F.Cu) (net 2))
 (segment (start 51.856989 76.159011) (end 53.048999 74.967001) (width 0.25) (layer F.Cu) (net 2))
 (segment (start 51.856989 81.239011) (end 51.856989 76.159011) (width 0.25) (layer F.Cu) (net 2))
 (segment (start 51.308 81.788) (end 51.856989 81.239011) (width 0.25) (layer F.Cu) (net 2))
 (segment (start 51.308 86.36) (end 51.308 81.788) (width 0.25) (layer F.Cu) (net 2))
 (segment (start 57.88 87.852) (end 71.024 87.852) (width 0.25) (layer F.Cu) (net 4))
 (segment (start 56.388 86.36) (end 57.88 87.852) (width 0.25) (layer F.Cu) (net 4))
 (segment (start 86.868 67.056) (end 86.868 65.532) (width 0.25) (layer B.Cu) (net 7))
 (segment (start 100.838 64.941998) (end 100.838 65.532) (width 0.25) (layer B.Cu) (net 7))
 (segment (start 100.353001 64.456999) (end 100.838 64.941998) (width 0.25) (layer B.Cu) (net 7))
 (segment (start 87.943001 64.456999) (end 100.353001 64.456999) (width 0.25) (layer B.Cu) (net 7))
 (segment (start 86.868 65.532) (end 87.943001 64.456999) (width 0.25) (layer B.Cu) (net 7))
 (segment (start 71.12 62.484) (end 76.2 62.484) (width 0.25) (layer F.Cu) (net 14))
 (segment (start 70.612 62.992) (end 71.12 62.484) (width 0.25) (layer F.Cu) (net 14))
 (segment (start 70.612 64.617002) (end 70.612 62.992) (width 0.25) (layer F.Cu) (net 14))
 (segment (start 70.210001 65.019001) (end 70.612 64.617002) (width 0.25) (layer F.Cu) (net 14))
 (segment (start 64.162998 62.992) (end 66.189999 65.019001) (width 0.25) (layer F.Cu) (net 14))
 (segment (start 45.212 62.992) (end 64.162998 62.992) (width 0.25) (layer F.Cu) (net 14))
 (segment (start 66.189999 65.019001) (end 70.210001 65.019001) (width 0.25) (layer F.Cu) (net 14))
 (segment (start 44.216 63.988) (end 45.212 62.992) (width 0.25) (layer F.Cu) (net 14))
 (segment (start 44.216 64.064) (end 44.216 63.988) (width 0.25) (layer F.Cu) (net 14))
 (segment (start 82.7 62.484) (end 76.2 62.484) (width 0.25) (layer F.Cu) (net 14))
 (segment (start 82.804 62.588) (end 82.7 62.484) (width 0.25) (layer F.Cu) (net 14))
 (segment (start 82.804 72.136) (end 82.804 62.588) (width 0.25) (layer F.Cu) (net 14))
 (segment (start 45.224 67.056) (end 67.056 67.056) (width 0.25) (layer F.Cu) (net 13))
 (segment (start 44.216 68.064) (end 45.224 67.056) (width 0.25) (layer F.Cu) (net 13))
 (segment (start 81.652 76.064) (end 82.804 77.216) (width 0.25) (layer F.Cu) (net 11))
 (segment (start 59.416 76.064) (end 81.652 76.064) (width 0.25) (layer F.Cu) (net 11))
 (segment (start 59.416 68.064) (end 63.492 68.064) (width 0.25) (layer F.Cu) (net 6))
 (segment (start 63.492 68.064) (end 64.008 68.58) (width 0.25) (layer F.Cu) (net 6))
 (segment (start 64.008 68.58) (end 67.197002 68.58) (width 0.25) (layer F.Cu) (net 6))
 (segment (start 78.122999 65.930999) (end 79.248 67.056) (width 0.25) (layer F.Cu) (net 6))
 (segment (start 69.846003 65.930999) (end 78.122999 65.930999) (width 0.25) (layer F.Cu) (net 6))
 (segment (start 67.197002 68.58) (end 69.846003 65.930999) (width 0.25) (layer F.Cu) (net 6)))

